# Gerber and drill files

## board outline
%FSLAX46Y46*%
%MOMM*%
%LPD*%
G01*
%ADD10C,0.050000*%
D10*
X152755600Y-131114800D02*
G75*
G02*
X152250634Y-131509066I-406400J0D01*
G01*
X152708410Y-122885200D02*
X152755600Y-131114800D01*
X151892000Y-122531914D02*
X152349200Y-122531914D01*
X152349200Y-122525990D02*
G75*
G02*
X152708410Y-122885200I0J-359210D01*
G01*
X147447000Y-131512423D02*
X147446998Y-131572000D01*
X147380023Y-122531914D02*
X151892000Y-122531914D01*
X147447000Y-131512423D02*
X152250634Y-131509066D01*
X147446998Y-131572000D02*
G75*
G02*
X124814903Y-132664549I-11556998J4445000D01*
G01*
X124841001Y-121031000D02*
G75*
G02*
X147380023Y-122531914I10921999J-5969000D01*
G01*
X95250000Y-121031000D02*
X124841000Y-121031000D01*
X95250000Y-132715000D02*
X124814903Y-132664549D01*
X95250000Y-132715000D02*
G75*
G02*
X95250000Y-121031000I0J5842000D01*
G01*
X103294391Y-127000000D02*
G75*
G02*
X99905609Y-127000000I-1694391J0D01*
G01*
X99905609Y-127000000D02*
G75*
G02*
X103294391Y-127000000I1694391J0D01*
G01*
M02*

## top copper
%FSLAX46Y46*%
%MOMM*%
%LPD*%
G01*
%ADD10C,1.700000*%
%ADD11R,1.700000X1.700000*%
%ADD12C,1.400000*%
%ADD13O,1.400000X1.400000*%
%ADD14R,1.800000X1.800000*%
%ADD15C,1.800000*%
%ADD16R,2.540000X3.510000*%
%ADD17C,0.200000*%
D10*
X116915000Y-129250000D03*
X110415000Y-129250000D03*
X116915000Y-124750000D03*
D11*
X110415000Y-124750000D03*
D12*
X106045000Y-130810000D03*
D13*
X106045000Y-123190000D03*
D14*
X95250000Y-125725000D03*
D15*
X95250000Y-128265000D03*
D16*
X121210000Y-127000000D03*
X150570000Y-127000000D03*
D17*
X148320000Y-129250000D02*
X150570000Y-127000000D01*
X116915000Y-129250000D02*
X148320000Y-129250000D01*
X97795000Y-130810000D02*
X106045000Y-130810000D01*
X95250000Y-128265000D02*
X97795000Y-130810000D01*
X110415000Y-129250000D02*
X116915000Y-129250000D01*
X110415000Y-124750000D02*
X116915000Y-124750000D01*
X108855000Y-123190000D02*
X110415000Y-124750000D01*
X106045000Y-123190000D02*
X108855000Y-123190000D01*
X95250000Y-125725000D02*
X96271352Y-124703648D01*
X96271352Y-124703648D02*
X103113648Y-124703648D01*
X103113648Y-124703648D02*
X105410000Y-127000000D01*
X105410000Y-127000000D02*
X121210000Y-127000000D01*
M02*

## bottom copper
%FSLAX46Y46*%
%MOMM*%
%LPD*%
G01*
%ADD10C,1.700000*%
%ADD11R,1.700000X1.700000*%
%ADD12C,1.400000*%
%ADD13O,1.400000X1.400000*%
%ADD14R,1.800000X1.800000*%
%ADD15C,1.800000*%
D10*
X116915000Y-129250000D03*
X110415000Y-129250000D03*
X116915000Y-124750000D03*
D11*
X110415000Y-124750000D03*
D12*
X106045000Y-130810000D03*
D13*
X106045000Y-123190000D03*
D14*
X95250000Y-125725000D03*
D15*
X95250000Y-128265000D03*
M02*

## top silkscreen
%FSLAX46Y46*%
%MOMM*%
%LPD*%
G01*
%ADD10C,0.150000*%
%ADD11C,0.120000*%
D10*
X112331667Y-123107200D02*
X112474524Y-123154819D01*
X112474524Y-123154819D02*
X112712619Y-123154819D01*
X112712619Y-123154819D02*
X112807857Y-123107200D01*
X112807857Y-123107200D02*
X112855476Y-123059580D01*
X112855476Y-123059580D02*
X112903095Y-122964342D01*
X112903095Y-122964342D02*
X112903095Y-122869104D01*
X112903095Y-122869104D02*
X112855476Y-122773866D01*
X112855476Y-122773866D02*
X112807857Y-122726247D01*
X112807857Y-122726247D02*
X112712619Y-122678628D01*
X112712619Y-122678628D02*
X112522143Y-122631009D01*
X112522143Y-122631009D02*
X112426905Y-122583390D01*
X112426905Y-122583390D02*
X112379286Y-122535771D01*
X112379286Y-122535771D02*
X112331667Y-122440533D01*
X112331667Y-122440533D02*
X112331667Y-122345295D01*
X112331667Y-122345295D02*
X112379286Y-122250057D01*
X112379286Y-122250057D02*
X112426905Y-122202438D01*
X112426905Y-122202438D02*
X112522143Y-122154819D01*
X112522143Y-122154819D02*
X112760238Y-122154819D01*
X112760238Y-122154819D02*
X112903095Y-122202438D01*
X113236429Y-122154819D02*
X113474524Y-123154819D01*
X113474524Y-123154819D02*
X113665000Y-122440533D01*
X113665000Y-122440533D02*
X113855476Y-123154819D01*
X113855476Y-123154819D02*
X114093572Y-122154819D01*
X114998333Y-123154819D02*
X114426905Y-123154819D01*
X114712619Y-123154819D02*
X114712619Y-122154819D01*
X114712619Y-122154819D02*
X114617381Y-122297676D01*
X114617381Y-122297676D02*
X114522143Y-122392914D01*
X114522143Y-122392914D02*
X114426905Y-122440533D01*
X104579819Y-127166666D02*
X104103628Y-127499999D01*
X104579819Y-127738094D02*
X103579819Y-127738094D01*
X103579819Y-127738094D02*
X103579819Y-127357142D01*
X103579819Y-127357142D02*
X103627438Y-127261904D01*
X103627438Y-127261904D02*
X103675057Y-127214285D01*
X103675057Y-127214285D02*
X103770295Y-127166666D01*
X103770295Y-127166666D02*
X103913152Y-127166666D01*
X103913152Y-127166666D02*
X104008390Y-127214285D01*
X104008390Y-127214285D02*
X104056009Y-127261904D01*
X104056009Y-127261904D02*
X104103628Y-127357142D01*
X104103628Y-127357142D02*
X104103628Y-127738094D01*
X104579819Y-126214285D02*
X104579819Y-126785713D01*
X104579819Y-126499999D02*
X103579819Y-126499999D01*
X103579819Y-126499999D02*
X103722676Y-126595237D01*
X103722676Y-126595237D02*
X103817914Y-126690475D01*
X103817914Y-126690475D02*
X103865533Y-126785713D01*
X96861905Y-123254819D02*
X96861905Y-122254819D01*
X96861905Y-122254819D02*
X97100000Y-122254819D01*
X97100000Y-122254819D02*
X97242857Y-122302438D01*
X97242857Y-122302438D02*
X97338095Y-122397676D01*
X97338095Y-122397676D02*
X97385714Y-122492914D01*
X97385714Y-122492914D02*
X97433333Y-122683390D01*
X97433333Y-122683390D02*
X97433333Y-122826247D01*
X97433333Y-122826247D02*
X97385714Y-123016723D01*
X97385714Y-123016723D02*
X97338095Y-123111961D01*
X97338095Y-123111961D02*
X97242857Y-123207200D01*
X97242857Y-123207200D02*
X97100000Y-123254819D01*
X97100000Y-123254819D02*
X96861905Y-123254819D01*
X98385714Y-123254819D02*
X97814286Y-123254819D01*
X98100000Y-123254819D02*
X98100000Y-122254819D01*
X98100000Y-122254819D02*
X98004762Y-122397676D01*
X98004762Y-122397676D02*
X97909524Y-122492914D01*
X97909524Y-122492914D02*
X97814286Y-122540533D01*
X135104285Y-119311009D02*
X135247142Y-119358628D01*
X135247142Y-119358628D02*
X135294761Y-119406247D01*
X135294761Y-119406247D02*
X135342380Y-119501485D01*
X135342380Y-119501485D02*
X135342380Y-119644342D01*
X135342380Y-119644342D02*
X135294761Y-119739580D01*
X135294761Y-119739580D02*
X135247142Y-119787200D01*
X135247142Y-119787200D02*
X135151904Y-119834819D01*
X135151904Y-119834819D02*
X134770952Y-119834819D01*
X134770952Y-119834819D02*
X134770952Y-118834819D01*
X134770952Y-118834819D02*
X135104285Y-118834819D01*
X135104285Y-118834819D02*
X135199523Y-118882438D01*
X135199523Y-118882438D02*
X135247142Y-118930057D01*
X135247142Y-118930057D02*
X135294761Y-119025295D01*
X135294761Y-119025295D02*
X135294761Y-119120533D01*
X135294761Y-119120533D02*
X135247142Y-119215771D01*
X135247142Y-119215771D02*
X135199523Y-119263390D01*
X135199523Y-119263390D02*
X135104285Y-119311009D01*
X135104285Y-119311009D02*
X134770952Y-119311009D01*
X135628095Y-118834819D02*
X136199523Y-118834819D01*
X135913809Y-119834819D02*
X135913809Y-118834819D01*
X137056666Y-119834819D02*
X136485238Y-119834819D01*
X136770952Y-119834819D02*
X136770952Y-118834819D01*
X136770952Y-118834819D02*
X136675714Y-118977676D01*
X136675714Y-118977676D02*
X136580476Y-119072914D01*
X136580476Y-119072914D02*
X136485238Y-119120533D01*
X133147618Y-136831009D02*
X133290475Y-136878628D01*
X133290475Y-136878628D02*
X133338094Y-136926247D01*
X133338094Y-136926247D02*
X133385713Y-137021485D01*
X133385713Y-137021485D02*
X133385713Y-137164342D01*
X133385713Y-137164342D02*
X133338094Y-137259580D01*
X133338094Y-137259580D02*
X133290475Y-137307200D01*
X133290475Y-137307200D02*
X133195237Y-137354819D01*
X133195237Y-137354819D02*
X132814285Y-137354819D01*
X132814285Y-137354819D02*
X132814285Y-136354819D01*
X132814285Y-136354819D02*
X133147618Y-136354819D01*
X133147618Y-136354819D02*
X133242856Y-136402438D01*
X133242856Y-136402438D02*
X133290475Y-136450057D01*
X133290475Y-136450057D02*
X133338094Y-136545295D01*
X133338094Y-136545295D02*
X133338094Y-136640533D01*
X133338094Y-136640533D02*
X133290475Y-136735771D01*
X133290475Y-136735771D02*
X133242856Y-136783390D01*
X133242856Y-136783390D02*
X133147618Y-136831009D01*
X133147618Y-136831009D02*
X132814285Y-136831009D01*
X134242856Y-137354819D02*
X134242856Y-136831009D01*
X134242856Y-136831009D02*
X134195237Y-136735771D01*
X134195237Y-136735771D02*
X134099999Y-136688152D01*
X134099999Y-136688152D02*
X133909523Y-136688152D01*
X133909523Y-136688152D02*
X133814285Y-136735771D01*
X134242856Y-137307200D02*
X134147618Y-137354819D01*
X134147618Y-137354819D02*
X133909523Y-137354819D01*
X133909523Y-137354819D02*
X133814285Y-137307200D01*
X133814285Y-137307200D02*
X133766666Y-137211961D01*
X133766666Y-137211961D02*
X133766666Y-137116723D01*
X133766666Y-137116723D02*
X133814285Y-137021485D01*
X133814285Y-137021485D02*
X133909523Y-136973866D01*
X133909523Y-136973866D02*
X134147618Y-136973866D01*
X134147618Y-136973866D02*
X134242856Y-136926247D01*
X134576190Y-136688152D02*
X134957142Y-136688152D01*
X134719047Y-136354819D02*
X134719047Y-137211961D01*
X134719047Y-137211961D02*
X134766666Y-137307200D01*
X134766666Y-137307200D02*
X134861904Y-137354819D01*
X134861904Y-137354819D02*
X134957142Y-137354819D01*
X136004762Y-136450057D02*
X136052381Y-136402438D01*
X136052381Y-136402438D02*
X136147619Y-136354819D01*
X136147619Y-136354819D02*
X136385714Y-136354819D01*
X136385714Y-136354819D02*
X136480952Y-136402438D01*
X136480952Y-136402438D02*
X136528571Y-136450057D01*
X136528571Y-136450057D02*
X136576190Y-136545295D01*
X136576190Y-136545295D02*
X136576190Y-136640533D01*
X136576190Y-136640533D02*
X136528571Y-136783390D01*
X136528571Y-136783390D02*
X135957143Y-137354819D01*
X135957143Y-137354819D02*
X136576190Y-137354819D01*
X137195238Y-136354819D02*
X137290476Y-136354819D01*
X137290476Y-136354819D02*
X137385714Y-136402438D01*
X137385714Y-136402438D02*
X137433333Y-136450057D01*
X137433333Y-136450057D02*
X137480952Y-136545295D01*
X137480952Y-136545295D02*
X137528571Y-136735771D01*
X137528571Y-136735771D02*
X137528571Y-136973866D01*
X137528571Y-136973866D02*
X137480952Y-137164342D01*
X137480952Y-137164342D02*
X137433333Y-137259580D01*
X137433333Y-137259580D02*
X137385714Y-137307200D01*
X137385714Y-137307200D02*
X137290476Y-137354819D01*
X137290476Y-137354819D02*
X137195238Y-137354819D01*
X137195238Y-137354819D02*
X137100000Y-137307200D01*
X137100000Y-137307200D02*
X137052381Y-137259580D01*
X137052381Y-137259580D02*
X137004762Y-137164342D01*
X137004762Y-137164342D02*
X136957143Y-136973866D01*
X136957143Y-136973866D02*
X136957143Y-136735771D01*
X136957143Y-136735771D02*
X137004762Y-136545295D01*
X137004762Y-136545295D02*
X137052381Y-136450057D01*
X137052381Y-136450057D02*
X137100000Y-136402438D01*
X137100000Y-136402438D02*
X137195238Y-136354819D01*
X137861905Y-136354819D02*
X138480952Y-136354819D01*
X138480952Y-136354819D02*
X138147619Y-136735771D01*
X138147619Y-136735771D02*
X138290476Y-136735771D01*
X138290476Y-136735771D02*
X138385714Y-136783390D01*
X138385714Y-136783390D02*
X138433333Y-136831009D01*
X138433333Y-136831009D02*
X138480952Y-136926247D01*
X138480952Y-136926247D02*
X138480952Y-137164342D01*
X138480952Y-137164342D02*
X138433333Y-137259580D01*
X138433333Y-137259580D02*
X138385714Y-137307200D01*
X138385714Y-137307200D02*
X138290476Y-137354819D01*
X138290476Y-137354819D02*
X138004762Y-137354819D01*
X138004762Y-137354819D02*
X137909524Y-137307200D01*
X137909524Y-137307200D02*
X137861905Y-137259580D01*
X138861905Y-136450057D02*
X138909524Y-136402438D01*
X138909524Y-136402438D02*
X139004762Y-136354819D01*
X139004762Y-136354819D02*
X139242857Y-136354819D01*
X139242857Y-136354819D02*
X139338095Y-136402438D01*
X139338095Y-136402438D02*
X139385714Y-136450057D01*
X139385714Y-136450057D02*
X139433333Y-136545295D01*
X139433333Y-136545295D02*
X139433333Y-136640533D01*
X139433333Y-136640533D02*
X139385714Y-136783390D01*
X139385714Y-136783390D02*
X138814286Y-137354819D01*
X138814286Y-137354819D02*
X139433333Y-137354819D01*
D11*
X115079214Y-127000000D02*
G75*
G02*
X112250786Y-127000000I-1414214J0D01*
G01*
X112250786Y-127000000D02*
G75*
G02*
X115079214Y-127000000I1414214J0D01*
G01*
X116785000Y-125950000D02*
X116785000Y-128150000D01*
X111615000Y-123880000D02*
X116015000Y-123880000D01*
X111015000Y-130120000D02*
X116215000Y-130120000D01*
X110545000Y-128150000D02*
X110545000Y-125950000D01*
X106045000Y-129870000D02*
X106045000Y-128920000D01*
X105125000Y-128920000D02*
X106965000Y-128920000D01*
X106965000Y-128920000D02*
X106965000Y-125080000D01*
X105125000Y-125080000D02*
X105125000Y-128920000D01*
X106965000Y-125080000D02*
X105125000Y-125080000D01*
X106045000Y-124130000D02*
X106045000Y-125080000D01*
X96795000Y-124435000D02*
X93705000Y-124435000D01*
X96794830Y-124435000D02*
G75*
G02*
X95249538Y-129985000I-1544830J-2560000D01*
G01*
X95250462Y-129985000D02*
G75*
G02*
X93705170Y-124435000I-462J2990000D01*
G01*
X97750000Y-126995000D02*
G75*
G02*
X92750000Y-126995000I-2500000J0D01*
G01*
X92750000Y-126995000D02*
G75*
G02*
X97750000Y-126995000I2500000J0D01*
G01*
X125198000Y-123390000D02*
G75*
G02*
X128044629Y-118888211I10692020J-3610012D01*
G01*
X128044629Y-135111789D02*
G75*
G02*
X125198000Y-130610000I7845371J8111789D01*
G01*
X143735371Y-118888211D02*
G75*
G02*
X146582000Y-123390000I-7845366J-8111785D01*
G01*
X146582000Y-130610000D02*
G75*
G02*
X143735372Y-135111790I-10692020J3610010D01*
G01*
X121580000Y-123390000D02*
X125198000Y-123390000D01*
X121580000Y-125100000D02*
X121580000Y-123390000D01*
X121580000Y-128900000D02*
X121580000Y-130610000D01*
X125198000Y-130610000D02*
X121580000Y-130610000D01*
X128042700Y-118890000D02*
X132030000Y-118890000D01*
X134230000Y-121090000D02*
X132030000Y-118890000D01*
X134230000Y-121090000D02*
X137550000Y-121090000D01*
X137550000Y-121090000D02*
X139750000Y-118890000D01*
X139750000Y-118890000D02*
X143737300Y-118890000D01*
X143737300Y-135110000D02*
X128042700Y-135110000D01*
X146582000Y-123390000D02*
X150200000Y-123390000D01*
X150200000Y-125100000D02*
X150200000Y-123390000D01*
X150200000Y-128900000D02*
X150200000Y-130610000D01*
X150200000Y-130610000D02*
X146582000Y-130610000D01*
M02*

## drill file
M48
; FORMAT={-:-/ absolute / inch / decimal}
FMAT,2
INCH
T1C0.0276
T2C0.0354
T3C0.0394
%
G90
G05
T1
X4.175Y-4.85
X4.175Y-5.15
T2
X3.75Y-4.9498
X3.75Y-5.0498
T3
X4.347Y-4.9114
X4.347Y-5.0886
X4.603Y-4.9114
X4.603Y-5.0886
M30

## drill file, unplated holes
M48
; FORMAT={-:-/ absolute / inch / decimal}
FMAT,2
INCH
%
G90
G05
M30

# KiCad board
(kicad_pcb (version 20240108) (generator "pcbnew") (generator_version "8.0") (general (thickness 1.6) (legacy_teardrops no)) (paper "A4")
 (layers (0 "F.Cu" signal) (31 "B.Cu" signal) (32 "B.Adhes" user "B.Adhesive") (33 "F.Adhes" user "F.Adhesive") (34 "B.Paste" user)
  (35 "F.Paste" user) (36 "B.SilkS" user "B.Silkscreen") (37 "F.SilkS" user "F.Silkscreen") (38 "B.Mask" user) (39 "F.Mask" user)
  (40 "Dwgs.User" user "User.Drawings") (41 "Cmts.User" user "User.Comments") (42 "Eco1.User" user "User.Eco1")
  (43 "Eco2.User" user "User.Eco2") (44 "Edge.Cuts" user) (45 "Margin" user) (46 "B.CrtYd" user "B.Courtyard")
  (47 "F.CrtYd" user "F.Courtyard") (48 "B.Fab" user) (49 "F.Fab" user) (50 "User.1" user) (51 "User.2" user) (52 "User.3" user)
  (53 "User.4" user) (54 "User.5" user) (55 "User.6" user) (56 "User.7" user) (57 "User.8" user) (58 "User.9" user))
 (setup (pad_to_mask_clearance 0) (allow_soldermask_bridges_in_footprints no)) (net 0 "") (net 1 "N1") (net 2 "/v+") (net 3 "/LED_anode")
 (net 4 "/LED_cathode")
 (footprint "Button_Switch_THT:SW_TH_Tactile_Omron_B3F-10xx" (layer "F.Cu") (at 110.415 124.75)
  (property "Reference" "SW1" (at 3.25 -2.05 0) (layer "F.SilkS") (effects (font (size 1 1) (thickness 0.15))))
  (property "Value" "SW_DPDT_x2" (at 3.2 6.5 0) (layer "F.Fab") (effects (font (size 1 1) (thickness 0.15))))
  (fp_line (start 0.13 3.4) (end 0.13 1.2) (stroke (width 0.12) (type solid)) (layer "F.SilkS"))
  (fp_line (start 0.6 5.37) (end 5.8 5.37) (stroke (width 0.12) (type solid)) (layer "F.SilkS"))
  (fp_line (start 1.2 -0.87) (end 5.6 -0.87) (stroke (width 0.12) (type solid)) (layer "F.SilkS"))
  (fp_line (start 6.37 1.2) (end 6.37 3.4) (stroke (width 0.12) (type solid)) (layer "F.SilkS"))
  (fp_circle (center 3.25 2.25) (end 4.25 3.25) (stroke (width 0.12) (type solid)) (fill none) (layer "F.SilkS"))
  (pad "1" thru_hole rect (at 0 0) (size 1.7 1.7) (drill 1) (layers "*.Cu" "*.Mask") (remove_unused_layers no) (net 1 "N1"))
  (pad "1" thru_hole circle (at 6.5 0) (size 1.7 1.7) (drill 1) (layers "*.Cu" "*.Mask") (remove_unused_layers no) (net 1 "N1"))
  (pad "2" thru_hole circle (at 0 4.5) (size 1.7 1.7) (drill 1) (layers "*.Cu" "*.Mask") (remove_unused_layers no) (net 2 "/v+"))
  (pad "2" thru_hole circle (at 6.5 4.5) (size 1.7 1.7) (drill 1) (layers "*.Cu" "*.Mask") (remove_unused_layers no) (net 2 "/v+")))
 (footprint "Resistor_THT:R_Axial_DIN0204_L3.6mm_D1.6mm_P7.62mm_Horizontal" (layer "F.Cu") (at 106.045 130.81 90)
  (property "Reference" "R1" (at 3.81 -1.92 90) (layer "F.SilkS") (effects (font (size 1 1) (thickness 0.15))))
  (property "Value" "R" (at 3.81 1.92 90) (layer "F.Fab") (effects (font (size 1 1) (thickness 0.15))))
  (fp_line (start 5.73 -0.92) (end 1.89 -0.92) (stroke (width 0.12) (type solid)) (layer "F.SilkS"))
  (fp_line (start 1.89 -0.92) (end 1.89 0.92) (stroke (width 0.12) (type solid)) (layer "F.SilkS"))
  (fp_line (start 6.68 0) (end 5.73 0) (stroke (width 0.12) (type solid)) (layer "F.SilkS"))
  (fp_line (start 0.94 0) (end 1.89 0) (stroke (width 0.12) (type solid)) (layer "F.SilkS"))
  (fp_line (start 5.73 0.92) (end 5.73 -0.92) (stroke (width 0.12) (type solid)) (layer "F.SilkS"))
  (fp_line (start 1.89 0.92) (end 5.73 0.92) (stroke (width 0.12) (type solid)) (layer "F.SilkS"))
  (pad "1" thru_hole circle (at 0 0 90) (size 1.4 1.4) (drill 0.7) (layers "*.Cu" "*.Mask") (remove_unused_layers no) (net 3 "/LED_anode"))
  (pad "2" thru_hole oval (at 7.62 0 90) (size 1.4 1.4) (drill 0.7) (layers "*.Cu" "*.Mask") (remove_unused_layers no) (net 1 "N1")))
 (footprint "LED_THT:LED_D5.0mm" (layer "F.Cu") (at 95.25 125.725 -90)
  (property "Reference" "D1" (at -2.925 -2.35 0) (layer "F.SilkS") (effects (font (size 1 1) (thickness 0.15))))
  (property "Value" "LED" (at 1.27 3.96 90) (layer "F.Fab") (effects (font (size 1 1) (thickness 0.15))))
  (fp_line (start -1.29 -1.545) (end -1.29 1.545) (stroke (width 0.12) (type solid)) (layer "F.SilkS"))
  (fp_arc (start 4.26 -0.000462) (mid 2.072002 2.880433) (end -1.29 1.54483) (stroke (width 0.12) (type solid)) (layer "F.SilkS"))
  (fp_arc (start -1.29 -1.54483) (mid 2.072002 -2.880433) (end 4.26 0.000462) (stroke (width 0.12) (type solid)) (layer "F.SilkS"))
  (fp_circle (center 1.27 0) (end 3.77 0) (stroke (width 0.12) (type solid)) (fill none) (layer "F.SilkS"))
  (pad "1" thru_hole rect (at 0 0 270) (size 1.8 1.8) (drill 0.9) (layers "*.Cu" "*.Mask") (remove_unused_layers no) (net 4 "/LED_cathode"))
  (pad "2" thru_hole circle (at 2.54 0 270) (size 1.8 1.8) (drill 0.9) (layers "*.Cu" "*.Mask") (remove_unused_layers no)
   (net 3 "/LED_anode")))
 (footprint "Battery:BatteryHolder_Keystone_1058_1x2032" (layer "F.Cu") (at 135.89 127 180)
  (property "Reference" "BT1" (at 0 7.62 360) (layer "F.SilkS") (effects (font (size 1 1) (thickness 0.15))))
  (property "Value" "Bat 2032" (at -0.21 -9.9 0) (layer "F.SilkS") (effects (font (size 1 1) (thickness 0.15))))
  (fp_line (start 14.31 3.61) (end 10.692 3.61) (stroke (width 0.12) (type solid)) (layer "F.SilkS"))
  (fp_line (start 14.31 1.9) (end 14.31 3.61) (stroke (width 0.12) (type solid)) (layer "F.SilkS"))
  (fp_line (start 14.31 -1.9) (end 14.31 -3.61) (stroke (width 0.12) (type solid)) (layer "F.SilkS"))
  (fp_line (start 10.692 -3.61) (end 14.31 -3.61) (stroke (width 0.12) (type solid)) (layer "F.SilkS"))
  (fp_line (start 7.8473 8.11) (end 3.86 8.11) (stroke (width 0.12) (type solid)) (layer "F.SilkS"))
  (fp_line (start 1.66 5.91) (end 3.86 8.11) (stroke (width 0.12) (type solid)) (layer "F.SilkS"))
  (fp_line (start 1.66 5.91) (end -1.66 5.91) (stroke (width 0.12) (type solid)) (layer "F.SilkS"))
  (fp_line (start -1.66 5.91) (end -3.86 8.11) (stroke (width 0.12) (type solid)) (layer "F.SilkS"))
  (fp_line (start -3.86 8.11) (end -7.8473 8.11) (stroke (width 0.12) (type solid)) (layer "F.SilkS"))
  (fp_line (start -7.8473 -8.11) (end 7.8473 -8.11) (stroke (width 0.12) (type solid)) (layer "F.SilkS"))
  (fp_line (start -10.692 3.61) (end -14.31 3.61) (stroke (width 0.12) (type solid)) (layer "F.SilkS"))
  (fp_line (start -14.31 1.9) (end -14.31 3.61) (stroke (width 0.12) (type solid)) (layer "F.SilkS"))
  (fp_line (start -14.31 -1.9) (end -14.31 -3.61) (stroke (width 0.12) (type solid)) (layer "F.SilkS"))
  (fp_line (start -14.31 -3.61) (end -10.692 -3.61) (stroke (width 0.12) (type solid)) (layer "F.SilkS"))
  (fp_arc (start 10.692 3.61) (mid 9.538084 6.031244) (end 7.845371 8.111789) (stroke (width 0.12) (type solid)) (layer "F.SilkS"))
  (fp_arc (start 7.845371 -8.111789) (mid 9.538085 -6.031244) (end 10.692 -3.61) (stroke (width 0.12) (type solid)) (layer "F.SilkS"))
  (fp_arc (start -7.845371 8.111789) (mid -9.538085 6.031244) (end -10.692 3.61) (stroke (width 0.12) (type solid)) (layer "F.SilkS"))
  (fp_arc (start -10.692 -3.61) (mid -9.538084 -6.031244) (end -7.845371 -8.111789) (stroke (width 0.12) (type solid)) (layer "F.SilkS"))
  (pad "1" smd rect (at -14.68 0 180) (size 2.54 3.51) (layers "F.Cu" "F.Paste" "F.Mask") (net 2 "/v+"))
  (pad "2" smd rect (at 14.68 0 180) (size 2.54 3.51) (layers "F.Cu" "F.Paste" "F.Mask") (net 4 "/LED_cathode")))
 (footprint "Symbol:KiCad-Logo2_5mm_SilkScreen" (layer "B.Cu") (at 135.509 127 180)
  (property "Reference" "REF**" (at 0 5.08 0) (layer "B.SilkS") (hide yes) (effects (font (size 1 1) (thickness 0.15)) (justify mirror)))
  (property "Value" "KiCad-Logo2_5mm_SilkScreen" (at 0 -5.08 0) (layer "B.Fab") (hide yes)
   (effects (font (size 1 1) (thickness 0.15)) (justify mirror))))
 (gr_line (start 147.447 131.512423) (end 152.250634 131.509066) (locked yes) (stroke (width 0.05) (type default)) (layer "Edge.Cuts"))
 (gr_arc (start 147.446998 131.572) (mid 136.487054 139.494933) (end 124.814903 132.664549) (locked yes)
  (stroke (width 0.05) (type default)) (layer "Edge.Cuts"))
 (gr_arc (start 152.7556 131.1148) (mid 152.599304 131.435127) (end 152.250634 131.509066) (locked yes) (stroke (width 0.05) (type default))
  (layer "Edge.Cuts"))
 (gr_arc (start 124.841001 121.031) (mid 136.590013 114.580859) (end 147.380023 122.531914) (locked yes)
  (stroke (width 0.05) (type default)) (layer "Edge.Cuts"))
 (gr_line (start 95.25 132.715) (end 124.814903 132.664549) (locked yes) (stroke (width 0.05) (type default)) (layer "Edge.Cuts"))
 (gr_line (start 151.892 122.531914) (end 152.3492 122.531914) (locked yes) (stroke (width 0.05) (type default)) (layer "Edge.Cuts"))
 (gr_line (start 95.25 121.031) (end 124.841 121.031) (locked yes) (stroke (width 0.05) (type default)) (layer "Edge.Cuts"))
 (gr_line (start 147.447 131.512423) (end 147.446998 131.572) (locked yes) (stroke (width 0.05) (type default)) (layer "Edge.Cuts"))
 (gr_line (start 152.70841 122.8852) (end 152.7556 131.1148) (locked yes) (stroke (width 0.05) (type default)) (layer "Edge.Cuts"))
 (gr_circle (center 101.6 127) (end 101.981 128.651) (stroke (width 0.05) (type default)) (fill none) (layer "Edge.Cuts"))
 (gr_line (start 147.380023 122.531914) (end 151.892 122.531914) (locked yes) (stroke (width 0.05) (type default)) (layer "Edge.Cuts"))
 (gr_arc (start 152.3492 122.52599) (mid 152.6032 122.6312) (end 152.70841 122.8852) (locked yes) (stroke (width 0.05) (type default))
  (layer "Edge.Cuts"))
 (gr_arc (start 95.25 132.715) (mid 89.408 126.873) (end 95.25 121.031) (locked yes) (stroke (width 0.05) (type default))
  (layer "Edge.Cuts"))
 (segment (start 110.415 129.25) (end 116.915 129.25) (width 0.2) (layer "F.Cu") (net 2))
 (segment (start 116.915 129.25) (end 148.32 129.25) (width 0.2) (layer "F.Cu") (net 2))
 (segment (start 148.32 129.25) (end 150.57 127) (width 0.2) (layer "F.Cu") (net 2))
 (segment (start 96.271352 124.703648) (end 103.113648 124.703648) (width 0.2) (layer "F.Cu") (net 4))
 (segment (start 105.41 127) (end 121.21 127) (width 0.2) (layer "F.Cu") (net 4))
 (segment (start 95.25 125.725) (end 96.271352 124.703648) (width 0.2) (layer "F.Cu") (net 4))
 (segment (start 103.113648 124.703648) (end 105.41 127) (width 0.2) (layer "F.Cu") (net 4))
 (segment (start 97.795 130.81) (end 106.045 130.81) (width 0.2) (layer "F.Cu") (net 3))
 (segment (start 95.25 128.265) (end 97.795 130.81) (width 0.2) (layer "F.Cu") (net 3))
 (segment (start 110.415 124.75) (end 116.915 124.75) (width 0.2) (layer "F.Cu") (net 1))
 (segment (start 108.855 123.19) (end 110.415 124.75) (width 0.2) (layer "F.Cu") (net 1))
 (segment (start 106.045 123.19) (end 108.855 123.19) (width 0.2) (layer "F.Cu") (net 1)))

